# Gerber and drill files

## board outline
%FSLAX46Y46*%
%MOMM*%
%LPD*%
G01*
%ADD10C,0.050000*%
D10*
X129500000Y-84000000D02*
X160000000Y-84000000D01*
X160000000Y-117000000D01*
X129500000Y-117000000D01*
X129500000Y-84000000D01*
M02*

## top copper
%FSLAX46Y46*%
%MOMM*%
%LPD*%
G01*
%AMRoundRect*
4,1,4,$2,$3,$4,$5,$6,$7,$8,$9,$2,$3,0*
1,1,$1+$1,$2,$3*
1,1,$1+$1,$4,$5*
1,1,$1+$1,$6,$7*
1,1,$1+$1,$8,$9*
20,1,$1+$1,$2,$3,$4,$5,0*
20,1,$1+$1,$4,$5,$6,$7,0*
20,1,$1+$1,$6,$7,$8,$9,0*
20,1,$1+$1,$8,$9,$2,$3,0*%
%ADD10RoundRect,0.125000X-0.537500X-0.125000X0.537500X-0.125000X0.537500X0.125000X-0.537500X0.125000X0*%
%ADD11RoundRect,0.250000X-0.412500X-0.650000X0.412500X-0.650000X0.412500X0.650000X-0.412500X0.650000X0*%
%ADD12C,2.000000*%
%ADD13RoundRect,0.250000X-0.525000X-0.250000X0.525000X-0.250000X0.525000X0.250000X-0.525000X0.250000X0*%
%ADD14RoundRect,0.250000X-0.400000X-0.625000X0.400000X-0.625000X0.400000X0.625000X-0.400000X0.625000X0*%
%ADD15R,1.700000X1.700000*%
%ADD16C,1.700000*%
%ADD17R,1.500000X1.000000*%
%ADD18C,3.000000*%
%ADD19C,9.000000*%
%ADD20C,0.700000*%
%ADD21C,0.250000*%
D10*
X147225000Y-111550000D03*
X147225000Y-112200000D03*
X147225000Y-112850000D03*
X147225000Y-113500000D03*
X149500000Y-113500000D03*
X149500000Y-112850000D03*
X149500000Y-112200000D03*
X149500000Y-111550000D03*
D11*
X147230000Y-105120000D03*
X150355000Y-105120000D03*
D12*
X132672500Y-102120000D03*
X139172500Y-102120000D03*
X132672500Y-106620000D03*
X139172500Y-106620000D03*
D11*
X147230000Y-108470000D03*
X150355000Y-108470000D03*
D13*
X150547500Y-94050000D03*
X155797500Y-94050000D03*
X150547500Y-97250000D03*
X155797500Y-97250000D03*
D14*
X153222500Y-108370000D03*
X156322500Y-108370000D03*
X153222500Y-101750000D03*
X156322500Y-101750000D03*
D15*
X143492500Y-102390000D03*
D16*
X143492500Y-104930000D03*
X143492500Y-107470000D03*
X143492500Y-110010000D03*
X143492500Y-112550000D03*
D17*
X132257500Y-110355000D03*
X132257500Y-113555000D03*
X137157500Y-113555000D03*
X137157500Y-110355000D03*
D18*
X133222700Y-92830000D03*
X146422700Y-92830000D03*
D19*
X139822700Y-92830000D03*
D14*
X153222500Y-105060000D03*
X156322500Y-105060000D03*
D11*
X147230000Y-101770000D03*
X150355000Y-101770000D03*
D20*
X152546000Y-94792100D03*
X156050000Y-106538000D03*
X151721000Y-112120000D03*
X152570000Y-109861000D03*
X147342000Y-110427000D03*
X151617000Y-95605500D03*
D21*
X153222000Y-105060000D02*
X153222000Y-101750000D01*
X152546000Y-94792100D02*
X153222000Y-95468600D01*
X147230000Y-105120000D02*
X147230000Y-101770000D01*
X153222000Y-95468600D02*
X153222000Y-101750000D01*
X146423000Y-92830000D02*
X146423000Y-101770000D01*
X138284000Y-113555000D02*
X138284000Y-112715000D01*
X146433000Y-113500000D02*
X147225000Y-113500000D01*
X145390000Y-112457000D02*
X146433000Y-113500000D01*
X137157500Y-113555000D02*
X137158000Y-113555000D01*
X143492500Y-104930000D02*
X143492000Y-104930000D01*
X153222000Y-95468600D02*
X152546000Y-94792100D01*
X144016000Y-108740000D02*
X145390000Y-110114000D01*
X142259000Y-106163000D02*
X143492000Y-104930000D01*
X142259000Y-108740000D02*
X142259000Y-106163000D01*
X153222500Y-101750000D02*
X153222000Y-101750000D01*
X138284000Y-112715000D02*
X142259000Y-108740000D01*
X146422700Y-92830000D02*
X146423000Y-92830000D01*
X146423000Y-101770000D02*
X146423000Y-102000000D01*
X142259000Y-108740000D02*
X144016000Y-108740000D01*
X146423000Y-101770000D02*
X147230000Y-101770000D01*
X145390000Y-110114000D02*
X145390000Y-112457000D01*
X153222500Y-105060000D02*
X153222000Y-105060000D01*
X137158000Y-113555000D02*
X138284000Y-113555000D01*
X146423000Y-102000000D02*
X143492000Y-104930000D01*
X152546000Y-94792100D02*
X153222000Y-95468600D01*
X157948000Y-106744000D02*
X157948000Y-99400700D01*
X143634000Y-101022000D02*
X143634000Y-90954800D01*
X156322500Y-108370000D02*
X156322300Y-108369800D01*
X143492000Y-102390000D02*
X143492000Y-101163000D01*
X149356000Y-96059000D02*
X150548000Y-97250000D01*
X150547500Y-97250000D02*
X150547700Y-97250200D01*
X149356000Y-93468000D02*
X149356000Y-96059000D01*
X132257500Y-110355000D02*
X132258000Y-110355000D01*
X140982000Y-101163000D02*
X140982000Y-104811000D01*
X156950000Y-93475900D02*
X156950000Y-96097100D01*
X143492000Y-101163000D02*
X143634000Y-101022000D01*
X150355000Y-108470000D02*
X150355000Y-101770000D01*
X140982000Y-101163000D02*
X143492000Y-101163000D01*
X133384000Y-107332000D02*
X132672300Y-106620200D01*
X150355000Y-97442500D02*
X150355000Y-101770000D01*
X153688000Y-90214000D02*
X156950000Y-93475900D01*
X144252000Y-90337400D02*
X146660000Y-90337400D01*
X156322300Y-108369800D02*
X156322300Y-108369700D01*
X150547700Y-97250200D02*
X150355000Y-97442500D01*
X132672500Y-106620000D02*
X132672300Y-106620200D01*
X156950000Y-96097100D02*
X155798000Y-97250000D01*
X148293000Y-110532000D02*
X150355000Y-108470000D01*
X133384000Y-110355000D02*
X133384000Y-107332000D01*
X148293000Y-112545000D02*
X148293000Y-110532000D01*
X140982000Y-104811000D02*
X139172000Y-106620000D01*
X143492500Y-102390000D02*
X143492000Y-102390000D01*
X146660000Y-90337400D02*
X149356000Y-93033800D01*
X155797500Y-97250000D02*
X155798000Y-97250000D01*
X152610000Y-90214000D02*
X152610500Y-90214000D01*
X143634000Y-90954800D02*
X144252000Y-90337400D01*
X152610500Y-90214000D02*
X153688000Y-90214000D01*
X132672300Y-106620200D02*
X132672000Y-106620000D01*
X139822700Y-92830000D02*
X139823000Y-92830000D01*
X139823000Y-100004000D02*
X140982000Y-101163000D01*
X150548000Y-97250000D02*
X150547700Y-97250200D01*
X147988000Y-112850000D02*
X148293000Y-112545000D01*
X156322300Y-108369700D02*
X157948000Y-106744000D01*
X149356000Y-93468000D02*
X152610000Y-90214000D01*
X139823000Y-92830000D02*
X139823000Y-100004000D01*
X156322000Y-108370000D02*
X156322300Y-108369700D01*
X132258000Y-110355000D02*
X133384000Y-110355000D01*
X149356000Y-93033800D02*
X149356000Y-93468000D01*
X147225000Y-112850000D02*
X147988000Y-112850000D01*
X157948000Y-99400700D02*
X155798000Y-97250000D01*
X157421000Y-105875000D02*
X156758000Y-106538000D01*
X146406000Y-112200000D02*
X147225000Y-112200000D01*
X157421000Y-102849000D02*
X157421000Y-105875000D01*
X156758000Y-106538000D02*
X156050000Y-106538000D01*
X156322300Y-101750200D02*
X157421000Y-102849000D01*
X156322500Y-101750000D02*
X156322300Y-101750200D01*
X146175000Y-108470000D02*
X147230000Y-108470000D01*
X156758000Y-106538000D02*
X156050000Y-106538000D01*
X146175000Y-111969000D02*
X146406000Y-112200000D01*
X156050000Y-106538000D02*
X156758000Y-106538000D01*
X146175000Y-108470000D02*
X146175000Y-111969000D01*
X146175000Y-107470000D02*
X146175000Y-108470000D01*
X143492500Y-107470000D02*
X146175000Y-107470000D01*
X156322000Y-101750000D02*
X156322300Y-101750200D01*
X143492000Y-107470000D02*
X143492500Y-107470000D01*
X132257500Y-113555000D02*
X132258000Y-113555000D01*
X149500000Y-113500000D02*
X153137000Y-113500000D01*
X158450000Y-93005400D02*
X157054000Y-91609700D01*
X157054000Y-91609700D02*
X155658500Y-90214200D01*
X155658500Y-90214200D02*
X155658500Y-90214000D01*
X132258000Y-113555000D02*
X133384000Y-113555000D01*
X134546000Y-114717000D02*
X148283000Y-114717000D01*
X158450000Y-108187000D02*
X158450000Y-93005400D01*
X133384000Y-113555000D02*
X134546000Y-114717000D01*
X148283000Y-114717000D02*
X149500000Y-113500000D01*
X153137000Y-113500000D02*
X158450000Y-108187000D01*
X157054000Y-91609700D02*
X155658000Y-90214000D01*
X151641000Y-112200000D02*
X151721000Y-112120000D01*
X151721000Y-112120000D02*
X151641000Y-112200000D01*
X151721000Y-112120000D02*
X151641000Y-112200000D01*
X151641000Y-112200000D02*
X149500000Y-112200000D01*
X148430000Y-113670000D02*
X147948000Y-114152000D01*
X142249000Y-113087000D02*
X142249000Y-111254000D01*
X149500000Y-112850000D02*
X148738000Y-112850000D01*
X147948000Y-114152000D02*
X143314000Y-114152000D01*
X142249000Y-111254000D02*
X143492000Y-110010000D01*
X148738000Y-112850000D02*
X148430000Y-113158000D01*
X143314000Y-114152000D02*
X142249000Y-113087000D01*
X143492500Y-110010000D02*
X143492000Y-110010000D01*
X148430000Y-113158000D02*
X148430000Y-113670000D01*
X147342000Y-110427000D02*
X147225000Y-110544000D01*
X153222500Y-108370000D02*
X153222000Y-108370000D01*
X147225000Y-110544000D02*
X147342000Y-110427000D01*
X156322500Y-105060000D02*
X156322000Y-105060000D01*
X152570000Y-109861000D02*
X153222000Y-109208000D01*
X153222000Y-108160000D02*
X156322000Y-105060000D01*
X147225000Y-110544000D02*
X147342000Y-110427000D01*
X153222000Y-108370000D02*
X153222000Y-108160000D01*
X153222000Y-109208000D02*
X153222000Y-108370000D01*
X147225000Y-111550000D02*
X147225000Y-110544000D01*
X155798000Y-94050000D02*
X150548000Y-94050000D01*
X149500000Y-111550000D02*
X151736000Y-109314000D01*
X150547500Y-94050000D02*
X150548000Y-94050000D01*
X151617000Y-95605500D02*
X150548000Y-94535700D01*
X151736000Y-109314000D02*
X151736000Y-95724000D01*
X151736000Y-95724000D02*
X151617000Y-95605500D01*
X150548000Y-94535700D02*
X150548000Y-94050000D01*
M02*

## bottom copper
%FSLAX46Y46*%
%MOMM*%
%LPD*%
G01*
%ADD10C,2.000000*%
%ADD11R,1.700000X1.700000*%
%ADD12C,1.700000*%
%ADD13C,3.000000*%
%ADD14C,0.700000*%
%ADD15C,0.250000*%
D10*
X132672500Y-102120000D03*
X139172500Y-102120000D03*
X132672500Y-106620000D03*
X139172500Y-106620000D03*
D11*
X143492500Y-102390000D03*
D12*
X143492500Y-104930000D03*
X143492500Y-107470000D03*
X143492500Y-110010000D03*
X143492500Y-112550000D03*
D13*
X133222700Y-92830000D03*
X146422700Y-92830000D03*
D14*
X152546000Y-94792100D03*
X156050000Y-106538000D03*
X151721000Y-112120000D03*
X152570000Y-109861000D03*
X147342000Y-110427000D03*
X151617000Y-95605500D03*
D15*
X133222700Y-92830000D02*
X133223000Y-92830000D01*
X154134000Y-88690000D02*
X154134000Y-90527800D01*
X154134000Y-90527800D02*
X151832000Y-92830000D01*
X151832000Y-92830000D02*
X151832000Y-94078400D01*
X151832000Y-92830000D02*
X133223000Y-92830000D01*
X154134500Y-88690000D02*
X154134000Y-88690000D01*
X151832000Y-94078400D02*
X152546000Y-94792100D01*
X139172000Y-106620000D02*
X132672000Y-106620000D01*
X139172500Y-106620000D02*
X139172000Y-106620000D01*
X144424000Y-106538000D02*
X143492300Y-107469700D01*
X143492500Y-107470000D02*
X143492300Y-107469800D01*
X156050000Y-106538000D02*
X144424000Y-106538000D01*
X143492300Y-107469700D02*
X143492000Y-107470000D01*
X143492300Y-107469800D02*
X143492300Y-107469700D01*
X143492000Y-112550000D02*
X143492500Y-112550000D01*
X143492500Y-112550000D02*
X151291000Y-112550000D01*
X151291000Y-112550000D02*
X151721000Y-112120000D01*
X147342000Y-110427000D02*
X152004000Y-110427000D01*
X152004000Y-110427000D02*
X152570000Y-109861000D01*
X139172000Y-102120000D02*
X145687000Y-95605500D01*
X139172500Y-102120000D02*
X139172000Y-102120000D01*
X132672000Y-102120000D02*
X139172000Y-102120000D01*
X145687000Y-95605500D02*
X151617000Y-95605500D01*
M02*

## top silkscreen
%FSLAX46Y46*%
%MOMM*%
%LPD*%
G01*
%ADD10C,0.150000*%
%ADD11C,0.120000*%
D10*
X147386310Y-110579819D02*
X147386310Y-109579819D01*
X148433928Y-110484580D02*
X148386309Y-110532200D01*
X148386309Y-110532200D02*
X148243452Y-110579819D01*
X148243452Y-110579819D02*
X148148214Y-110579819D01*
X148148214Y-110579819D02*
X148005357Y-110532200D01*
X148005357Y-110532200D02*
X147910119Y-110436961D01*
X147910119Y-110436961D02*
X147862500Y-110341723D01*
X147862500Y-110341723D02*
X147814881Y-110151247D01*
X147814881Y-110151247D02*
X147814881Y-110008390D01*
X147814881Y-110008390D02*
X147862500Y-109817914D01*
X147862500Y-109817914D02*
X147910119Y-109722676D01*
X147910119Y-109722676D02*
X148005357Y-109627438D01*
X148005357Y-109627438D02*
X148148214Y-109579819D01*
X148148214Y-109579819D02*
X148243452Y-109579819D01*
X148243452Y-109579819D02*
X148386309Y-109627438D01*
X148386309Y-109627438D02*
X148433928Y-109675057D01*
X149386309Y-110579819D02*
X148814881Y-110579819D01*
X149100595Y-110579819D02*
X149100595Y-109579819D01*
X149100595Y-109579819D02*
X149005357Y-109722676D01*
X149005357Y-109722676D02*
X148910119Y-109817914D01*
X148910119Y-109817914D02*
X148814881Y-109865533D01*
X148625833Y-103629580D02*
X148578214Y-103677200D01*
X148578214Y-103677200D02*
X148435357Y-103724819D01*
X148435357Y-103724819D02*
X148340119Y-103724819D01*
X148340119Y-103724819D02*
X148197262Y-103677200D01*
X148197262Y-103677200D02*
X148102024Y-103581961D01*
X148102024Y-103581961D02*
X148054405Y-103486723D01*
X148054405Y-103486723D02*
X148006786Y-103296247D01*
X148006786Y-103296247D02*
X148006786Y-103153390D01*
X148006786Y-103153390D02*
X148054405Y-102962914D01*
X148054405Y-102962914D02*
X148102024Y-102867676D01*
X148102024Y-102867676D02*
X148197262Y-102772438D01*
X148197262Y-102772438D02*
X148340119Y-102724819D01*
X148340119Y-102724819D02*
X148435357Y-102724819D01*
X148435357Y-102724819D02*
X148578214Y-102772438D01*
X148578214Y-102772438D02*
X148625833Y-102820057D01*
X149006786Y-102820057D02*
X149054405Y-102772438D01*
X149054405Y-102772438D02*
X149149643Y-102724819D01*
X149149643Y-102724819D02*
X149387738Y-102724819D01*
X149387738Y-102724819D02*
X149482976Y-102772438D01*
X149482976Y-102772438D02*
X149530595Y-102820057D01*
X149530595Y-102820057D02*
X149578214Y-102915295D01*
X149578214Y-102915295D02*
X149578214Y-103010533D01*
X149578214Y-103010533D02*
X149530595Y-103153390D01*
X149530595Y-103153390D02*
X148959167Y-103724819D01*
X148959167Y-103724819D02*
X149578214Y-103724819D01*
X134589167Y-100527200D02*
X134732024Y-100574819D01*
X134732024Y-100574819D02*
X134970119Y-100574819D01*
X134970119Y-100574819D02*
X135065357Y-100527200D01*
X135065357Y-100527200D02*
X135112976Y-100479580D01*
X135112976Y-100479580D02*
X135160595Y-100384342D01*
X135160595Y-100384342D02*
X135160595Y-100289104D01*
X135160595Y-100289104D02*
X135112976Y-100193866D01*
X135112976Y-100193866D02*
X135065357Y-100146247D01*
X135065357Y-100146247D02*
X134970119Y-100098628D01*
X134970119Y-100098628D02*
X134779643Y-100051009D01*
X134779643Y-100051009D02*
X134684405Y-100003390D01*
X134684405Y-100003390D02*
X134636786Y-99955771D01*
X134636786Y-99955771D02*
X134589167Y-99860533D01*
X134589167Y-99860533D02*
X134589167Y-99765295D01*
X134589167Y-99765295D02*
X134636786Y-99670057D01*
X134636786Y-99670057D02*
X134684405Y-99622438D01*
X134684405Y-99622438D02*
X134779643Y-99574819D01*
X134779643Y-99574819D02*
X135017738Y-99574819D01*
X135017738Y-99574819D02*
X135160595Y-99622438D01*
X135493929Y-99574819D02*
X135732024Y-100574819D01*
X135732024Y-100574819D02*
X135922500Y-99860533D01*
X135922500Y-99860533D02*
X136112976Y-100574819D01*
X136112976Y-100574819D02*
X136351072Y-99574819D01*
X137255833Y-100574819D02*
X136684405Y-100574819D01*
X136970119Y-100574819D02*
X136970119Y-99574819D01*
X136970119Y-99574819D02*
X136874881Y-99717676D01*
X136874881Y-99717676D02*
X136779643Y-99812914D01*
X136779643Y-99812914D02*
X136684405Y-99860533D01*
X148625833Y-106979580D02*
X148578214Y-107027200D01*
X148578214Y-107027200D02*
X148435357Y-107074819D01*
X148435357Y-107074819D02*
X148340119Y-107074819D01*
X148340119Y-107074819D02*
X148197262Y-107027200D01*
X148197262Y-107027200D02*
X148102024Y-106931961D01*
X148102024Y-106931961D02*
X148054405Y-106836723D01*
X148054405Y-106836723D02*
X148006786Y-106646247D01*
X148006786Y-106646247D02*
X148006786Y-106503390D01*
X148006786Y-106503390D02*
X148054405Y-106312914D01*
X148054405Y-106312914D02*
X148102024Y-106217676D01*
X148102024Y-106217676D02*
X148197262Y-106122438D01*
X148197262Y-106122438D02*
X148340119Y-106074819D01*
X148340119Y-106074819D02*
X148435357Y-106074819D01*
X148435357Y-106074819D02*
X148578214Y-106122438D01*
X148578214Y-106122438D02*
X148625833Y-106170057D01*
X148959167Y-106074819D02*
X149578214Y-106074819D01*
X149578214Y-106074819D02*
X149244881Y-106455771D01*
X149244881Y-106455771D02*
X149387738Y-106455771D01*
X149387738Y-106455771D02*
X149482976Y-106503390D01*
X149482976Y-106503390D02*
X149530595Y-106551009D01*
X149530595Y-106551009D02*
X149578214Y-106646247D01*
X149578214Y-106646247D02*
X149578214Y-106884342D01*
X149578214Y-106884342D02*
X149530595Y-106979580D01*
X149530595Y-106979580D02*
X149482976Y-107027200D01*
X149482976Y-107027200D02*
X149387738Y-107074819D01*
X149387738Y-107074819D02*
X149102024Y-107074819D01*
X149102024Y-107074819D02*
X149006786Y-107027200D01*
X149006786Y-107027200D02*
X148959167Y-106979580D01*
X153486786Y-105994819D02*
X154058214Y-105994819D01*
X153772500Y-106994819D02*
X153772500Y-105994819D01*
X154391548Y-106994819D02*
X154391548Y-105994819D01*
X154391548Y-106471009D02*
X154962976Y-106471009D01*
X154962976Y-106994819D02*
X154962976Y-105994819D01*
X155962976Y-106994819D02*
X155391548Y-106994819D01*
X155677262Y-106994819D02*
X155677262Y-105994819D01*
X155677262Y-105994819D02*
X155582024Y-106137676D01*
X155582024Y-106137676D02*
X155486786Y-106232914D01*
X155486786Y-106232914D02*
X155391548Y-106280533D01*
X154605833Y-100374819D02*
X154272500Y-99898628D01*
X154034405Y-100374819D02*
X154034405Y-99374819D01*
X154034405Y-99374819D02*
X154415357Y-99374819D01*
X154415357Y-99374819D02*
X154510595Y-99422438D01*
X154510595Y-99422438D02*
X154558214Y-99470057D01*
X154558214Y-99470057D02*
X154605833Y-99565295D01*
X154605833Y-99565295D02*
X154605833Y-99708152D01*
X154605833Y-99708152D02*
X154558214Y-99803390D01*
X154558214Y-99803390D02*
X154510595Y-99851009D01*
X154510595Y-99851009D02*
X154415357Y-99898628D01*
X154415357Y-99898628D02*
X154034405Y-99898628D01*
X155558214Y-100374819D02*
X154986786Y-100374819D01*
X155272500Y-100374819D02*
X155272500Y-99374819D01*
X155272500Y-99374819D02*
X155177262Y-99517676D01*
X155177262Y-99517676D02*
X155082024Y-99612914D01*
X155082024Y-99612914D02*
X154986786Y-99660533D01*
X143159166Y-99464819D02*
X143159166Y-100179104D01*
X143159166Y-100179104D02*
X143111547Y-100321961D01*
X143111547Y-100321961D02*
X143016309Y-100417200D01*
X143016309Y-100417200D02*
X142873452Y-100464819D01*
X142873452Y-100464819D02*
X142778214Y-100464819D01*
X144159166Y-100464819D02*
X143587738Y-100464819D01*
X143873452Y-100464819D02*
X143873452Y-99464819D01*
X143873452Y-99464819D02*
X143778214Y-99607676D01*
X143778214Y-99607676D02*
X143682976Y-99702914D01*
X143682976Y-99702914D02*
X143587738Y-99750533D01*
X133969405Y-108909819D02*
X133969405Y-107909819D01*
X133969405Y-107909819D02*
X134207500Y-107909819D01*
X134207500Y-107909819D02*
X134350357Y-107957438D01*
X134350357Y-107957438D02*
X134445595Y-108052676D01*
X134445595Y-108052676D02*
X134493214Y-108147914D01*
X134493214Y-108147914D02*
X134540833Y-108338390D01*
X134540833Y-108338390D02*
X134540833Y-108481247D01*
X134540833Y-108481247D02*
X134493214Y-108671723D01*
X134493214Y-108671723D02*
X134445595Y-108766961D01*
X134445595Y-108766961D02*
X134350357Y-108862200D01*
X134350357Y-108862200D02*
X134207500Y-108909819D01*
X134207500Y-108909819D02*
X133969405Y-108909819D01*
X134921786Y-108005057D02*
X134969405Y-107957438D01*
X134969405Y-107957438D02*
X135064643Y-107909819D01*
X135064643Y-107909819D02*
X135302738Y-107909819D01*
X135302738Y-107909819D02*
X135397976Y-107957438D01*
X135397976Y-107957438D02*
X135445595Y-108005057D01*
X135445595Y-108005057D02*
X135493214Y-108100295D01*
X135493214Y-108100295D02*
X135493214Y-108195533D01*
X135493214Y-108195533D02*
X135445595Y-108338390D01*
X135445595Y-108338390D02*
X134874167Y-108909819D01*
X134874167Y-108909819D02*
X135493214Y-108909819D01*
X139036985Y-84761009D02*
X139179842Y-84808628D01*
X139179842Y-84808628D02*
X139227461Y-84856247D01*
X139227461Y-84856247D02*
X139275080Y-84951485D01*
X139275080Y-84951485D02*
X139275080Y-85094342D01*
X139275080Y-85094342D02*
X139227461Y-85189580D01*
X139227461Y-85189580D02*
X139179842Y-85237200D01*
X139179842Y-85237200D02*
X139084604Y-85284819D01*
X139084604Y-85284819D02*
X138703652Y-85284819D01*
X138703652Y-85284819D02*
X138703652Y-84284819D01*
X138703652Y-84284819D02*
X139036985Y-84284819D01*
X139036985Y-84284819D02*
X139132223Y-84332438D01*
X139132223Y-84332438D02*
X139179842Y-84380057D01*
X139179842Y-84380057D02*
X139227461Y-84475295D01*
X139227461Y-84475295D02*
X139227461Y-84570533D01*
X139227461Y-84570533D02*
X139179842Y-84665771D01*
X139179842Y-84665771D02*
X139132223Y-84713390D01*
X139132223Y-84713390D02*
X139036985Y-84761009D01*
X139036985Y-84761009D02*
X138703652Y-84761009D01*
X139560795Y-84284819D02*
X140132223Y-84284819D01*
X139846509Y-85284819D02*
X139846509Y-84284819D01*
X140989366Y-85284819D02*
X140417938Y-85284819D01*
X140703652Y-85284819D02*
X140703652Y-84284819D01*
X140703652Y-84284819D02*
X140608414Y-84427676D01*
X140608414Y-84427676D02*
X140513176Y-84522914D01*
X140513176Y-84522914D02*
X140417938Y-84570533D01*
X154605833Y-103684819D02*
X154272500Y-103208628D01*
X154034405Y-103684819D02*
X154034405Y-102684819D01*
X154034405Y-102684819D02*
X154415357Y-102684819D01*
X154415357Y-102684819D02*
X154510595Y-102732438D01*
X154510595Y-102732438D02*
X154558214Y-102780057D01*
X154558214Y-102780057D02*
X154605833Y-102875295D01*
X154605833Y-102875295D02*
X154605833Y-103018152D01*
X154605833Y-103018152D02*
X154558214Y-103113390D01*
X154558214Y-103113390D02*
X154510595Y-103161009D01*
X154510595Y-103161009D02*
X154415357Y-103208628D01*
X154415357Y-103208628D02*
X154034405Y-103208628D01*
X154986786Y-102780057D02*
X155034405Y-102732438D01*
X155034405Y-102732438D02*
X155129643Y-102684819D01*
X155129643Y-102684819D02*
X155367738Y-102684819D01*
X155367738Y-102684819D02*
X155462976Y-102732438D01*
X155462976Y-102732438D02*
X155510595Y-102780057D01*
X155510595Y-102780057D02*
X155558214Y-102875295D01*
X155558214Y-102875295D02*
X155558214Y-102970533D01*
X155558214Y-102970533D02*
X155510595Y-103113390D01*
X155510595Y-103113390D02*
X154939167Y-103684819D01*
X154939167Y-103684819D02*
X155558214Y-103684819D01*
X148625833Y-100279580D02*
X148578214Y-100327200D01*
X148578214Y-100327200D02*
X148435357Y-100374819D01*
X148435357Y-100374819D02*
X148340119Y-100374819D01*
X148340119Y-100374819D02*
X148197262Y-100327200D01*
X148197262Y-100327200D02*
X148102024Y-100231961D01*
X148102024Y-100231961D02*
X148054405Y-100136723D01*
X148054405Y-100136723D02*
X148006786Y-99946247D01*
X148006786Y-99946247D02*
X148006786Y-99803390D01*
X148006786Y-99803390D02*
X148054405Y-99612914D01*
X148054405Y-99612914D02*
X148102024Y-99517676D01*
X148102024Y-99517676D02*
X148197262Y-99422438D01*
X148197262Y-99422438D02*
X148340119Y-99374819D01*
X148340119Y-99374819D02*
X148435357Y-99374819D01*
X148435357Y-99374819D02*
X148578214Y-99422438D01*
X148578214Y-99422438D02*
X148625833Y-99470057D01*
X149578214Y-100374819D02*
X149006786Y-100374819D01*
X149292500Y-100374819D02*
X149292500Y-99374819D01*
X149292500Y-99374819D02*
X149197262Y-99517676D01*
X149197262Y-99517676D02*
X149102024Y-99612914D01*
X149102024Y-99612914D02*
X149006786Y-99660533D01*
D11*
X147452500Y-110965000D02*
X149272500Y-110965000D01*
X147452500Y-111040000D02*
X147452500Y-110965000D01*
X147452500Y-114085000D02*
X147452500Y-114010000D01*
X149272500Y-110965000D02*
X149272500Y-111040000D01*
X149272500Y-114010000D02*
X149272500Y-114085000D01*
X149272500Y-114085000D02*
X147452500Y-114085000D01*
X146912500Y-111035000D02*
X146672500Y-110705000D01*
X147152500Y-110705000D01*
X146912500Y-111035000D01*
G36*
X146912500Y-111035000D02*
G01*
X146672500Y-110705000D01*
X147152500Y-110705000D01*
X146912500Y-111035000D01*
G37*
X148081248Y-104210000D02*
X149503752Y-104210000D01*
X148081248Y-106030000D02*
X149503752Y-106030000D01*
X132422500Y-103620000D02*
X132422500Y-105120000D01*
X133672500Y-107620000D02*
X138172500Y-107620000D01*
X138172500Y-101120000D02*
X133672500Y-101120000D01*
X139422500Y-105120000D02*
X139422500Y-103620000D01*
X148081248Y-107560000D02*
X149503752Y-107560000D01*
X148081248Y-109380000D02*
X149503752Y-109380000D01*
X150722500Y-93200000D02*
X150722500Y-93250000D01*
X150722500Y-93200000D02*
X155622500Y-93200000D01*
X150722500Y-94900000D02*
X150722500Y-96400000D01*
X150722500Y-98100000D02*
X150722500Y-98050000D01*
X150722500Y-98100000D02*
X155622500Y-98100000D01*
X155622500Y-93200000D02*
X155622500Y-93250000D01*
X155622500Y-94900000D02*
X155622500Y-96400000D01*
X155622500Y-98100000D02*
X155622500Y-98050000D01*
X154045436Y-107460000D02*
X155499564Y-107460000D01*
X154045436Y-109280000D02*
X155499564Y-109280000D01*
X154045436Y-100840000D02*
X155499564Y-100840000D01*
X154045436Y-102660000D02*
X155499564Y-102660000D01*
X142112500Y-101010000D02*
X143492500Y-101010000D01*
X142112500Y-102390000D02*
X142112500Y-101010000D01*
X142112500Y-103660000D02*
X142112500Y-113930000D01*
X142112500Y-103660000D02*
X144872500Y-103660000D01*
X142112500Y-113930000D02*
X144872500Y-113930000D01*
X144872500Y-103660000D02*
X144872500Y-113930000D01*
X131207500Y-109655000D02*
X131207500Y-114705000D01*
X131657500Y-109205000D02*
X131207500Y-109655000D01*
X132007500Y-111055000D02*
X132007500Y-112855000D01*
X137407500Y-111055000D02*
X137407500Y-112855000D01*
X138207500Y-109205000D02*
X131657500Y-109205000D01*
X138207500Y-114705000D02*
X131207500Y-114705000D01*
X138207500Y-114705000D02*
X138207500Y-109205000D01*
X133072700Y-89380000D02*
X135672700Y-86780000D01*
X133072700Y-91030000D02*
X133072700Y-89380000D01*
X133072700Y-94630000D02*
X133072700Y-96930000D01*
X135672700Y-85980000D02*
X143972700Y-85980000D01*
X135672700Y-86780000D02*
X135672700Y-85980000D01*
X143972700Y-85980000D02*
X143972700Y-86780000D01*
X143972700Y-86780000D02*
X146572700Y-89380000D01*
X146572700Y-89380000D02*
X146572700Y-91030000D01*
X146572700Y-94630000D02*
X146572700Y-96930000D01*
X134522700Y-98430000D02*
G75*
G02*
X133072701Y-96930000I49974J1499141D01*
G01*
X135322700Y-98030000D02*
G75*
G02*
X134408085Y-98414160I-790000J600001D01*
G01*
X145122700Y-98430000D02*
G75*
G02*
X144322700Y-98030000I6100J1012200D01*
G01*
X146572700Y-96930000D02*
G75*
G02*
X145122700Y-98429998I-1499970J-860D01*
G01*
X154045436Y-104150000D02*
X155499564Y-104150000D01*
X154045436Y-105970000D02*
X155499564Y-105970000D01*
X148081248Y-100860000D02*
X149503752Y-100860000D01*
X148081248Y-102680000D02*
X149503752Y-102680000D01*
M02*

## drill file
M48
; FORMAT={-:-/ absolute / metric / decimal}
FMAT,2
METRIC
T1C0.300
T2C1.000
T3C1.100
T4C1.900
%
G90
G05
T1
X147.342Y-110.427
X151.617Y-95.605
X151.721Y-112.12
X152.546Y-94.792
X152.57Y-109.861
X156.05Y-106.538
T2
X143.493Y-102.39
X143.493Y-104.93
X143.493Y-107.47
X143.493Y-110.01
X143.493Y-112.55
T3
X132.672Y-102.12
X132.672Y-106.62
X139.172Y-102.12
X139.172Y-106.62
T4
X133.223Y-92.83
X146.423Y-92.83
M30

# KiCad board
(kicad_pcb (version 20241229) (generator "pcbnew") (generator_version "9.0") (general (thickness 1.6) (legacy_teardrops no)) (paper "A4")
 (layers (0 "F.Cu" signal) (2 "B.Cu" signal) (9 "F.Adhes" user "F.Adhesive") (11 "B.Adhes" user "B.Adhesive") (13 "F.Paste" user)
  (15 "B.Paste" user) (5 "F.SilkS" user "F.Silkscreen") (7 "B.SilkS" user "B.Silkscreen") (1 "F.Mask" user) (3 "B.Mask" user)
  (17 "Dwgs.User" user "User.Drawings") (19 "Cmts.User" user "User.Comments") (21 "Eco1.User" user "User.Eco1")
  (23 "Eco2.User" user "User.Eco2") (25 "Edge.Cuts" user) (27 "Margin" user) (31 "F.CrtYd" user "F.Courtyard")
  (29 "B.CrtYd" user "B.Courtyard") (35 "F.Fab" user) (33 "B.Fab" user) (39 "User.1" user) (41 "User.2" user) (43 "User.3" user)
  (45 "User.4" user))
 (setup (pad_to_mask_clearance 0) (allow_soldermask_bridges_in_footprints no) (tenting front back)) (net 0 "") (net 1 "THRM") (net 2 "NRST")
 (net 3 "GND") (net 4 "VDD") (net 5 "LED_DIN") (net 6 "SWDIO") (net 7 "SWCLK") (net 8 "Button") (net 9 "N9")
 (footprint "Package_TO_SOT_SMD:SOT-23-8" (layer "F.Cu") (at 148.3625 112.525)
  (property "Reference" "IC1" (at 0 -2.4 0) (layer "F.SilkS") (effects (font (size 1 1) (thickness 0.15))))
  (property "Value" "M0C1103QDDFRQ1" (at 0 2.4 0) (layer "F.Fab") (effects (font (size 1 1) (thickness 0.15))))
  (fp_line (start -0.91 -1.56) (end 0.91 -1.56) (stroke (width 0.12) (type solid)) (layer "F.SilkS"))
  (fp_line (start -0.91 -1.485) (end -0.91 -1.56) (stroke (width 0.12) (type solid)) (layer "F.SilkS"))
  (fp_line (start -0.91 1.56) (end -0.91 1.485) (stroke (width 0.12) (type solid)) (layer "F.SilkS"))
  (fp_line (start 0.91 -1.56) (end 0.91 -1.485) (stroke (width 0.12) (type solid)) (layer "F.SilkS"))
  (fp_line (start 0.91 1.485) (end 0.91 1.56) (stroke (width 0.12) (type solid)) (layer "F.SilkS"))
  (fp_line (start 0.91 1.56) (end -0.91 1.56) (stroke (width 0.12) (type solid)) (layer "F.SilkS"))
  (fp_poly (pts (xy -1.45 -1.49) (xy -1.69 -1.82) (xy -1.21 -1.82)) (stroke (width 0.12) (type solid)) (fill yes) (layer "F.SilkS"))
  (pad "1" smd roundrect (at -1.1375 -0.975) (size 1.325 0.5) (layers "F.Cu" "F.Mask" "F.Paste") (roundrect_rratio 0.25) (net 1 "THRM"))
  (pad "2" smd roundrect (at -1.1375 -0.325) (size 1.325 0.5) (layers "F.Cu" "F.Mask" "F.Paste") (roundrect_rratio 0.25) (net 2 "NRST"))
  (pad "3" smd roundrect (at -1.1375 0.325) (size 1.325 0.5) (layers "F.Cu" "F.Mask" "F.Paste") (roundrect_rratio 0.25) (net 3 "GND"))
  (pad "4" smd roundrect (at -1.1375 0.975) (size 1.325 0.5) (layers "F.Cu" "F.Mask" "F.Paste") (roundrect_rratio 0.25) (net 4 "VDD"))
  (pad "5" smd roundrect (at 1.1375 0.975) (size 1.325 0.5) (layers "F.Cu" "F.Mask" "F.Paste") (roundrect_rratio 0.25) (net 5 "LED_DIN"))
  (pad "6" smd roundrect (at 1.1375 0.325) (size 1.325 0.5) (layers "F.Cu" "F.Mask" "F.Paste") (roundrect_rratio 0.25) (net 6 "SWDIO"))
  (pad "7" smd roundrect (at 1.1375 -0.325) (size 1.325 0.5) (layers "F.Cu" "F.Mask" "F.Paste") (roundrect_rratio 0.25) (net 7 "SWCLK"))
  (pad "8" smd roundrect (at 1.1375 -0.975) (size 1.325 0.5) (layers "F.Cu" "F.Mask" "F.Paste") (roundrect_rratio 0.25) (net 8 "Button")))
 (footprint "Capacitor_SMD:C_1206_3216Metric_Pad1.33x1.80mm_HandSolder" (layer "F.Cu") (at 148.7925 105.12)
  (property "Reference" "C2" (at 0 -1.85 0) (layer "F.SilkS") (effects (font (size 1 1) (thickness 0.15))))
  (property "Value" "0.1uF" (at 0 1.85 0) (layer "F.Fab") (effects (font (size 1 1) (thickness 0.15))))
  (fp_line (start -0.711252 -0.91) (end 0.711252 -0.91) (stroke (width 0.12) (type solid)) (layer "F.SilkS"))
  (fp_line (start -0.711252 0.91) (end 0.711252 0.91) (stroke (width 0.12) (type solid)) (layer "F.SilkS"))
  (pad "1" smd roundrect (at -1.5625 0) (size 1.325 1.8) (layers "F.Cu" "F.Mask" "F.Paste") (roundrect_rratio 0.188679) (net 4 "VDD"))
  (pad "2" smd roundrect (at 1.5625 0) (size 1.325 1.8) (layers "F.Cu" "F.Mask" "F.Paste") (roundrect_rratio 0.188679) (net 3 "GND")))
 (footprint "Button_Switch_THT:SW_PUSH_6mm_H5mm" (layer "F.Cu") (at 132.6725 102.12)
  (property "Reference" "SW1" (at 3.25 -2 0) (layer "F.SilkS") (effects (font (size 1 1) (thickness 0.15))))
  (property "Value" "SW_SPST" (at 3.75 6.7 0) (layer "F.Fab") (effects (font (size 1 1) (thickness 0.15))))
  (fp_line (start -0.25 1.5) (end -0.25 3) (stroke (width 0.12) (type solid)) (layer "F.SilkS"))
  (fp_line (start 1 5.5) (end 5.5 5.5) (stroke (width 0.12) (type solid)) (layer "F.SilkS"))
  (fp_line (start 5.5 -1) (end 1 -1) (stroke (width 0.12) (type solid)) (layer "F.SilkS"))
  (fp_line (start 6.75 3) (end 6.75 1.5) (stroke (width 0.12) (type solid)) (layer "F.SilkS"))
  (pad "1" thru_hole circle (at 0 0 90) (size 2 2) (drill 1.1) (layers "*.Cu" "*.Mask") (remove_unused_layers no) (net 8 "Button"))
  (pad "1" thru_hole circle (at 6.5 0 90) (size 2 2) (drill 1.1) (layers "*.Cu" "*.Mask") (remove_unused_layers no) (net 8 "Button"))
  (pad "2" thru_hole circle (at 0 4.5 90) (size 2 2) (drill 1.1) (layers "*.Cu" "*.Mask") (remove_unused_layers no) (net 3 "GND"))
  (pad "2" thru_hole circle (at 6.5 4.5 90) (size 2 2) (drill 1.1) (layers "*.Cu" "*.Mask") (remove_unused_layers no) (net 3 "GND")))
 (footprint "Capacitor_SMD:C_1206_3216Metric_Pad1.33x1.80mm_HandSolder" (layer "F.Cu") (at 148.7925 108.47)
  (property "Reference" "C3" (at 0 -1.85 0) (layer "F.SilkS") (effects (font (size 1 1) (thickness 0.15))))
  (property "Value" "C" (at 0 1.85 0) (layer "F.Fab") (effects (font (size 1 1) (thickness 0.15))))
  (fp_line (start -0.711252 -0.91) (end 0.711252 -0.91) (stroke (width 0.12) (type solid)) (layer "F.SilkS"))
  (fp_line (start -0.711252 0.91) (end 0.711252 0.91) (stroke (width 0.12) (type solid)) (layer "F.SilkS"))
  (pad "1" smd roundrect (at -1.5625 0) (size 1.325 1.8) (layers "F.Cu" "F.Mask" "F.Paste") (roundrect_rratio 0.188679) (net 2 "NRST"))
  (pad "2" smd roundrect (at 1.5625 0) (size 1.325 1.8) (layers "F.Cu" "F.Mask" "F.Paste") (roundrect_rratio 0.188679) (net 3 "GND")))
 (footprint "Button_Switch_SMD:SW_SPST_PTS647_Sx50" (layer "F.Cu") (at 153.1725 95.65)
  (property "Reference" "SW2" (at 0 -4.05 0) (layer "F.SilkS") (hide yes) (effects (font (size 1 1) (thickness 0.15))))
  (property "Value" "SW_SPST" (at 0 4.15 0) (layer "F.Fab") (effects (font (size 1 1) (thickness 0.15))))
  (fp_line (start -2.45 -2.45) (end -2.45 -2.4) (stroke (width 0.12) (type solid)) (layer "F.SilkS"))
  (fp_line (start -2.45 -2.45) (end 2.45 -2.45) (stroke (width 0.12) (type solid)) (layer "F.SilkS"))
  (fp_line (start -2.45 -0.75) (end -2.45 0.75) (stroke (width 0.12) (type solid)) (layer "F.SilkS"))
  (fp_line (start -2.45 2.45) (end -2.45 2.4) (stroke (width 0.12) (type solid)) (layer "F.SilkS"))
  (fp_line (start -2.45 2.45) (end 2.45 2.45) (stroke (width 0.12) (type solid)) (layer "F.SilkS"))
  (fp_line (start 2.45 -2.45) (end 2.45 -2.4) (stroke (width 0.12) (type solid)) (layer "F.SilkS"))
  (fp_line (start 2.45 -0.75) (end 2.45 0.75) (stroke (width 0.12) (type solid)) (layer "F.SilkS"))
  (fp_line (start 2.45 2.45) (end 2.45 2.4) (stroke (width 0.12) (type solid)) (layer "F.SilkS"))
  (pad "1" smd roundrect (at -2.625 -1.6) (size 1.55 1) (layers "F.Cu" "F.Mask" "F.Paste") (roundrect_rratio 0.25) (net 8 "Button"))
  (pad "1" smd roundrect (at 2.625 -1.6) (size 1.55 1) (layers "F.Cu" "F.Mask" "F.Paste") (roundrect_rratio 0.25) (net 8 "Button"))
  (pad "2" smd roundrect (at -2.625 1.6) (size 1.55 1) (layers "F.Cu" "F.Mask" "F.Paste") (roundrect_rratio 0.25) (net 3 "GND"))
  (pad "2" smd roundrect (at 2.625 1.6) (size 1.55 1) (layers "F.Cu" "F.Mask" "F.Paste") (roundrect_rratio 0.25) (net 3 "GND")))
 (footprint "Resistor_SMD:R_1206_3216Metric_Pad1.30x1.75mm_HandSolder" (layer "F.Cu") (at 154.7725 108.37)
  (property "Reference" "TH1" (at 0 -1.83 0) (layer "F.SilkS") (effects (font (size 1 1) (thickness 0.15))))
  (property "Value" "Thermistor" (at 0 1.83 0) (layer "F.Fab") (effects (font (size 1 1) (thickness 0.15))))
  (fp_line (start -0.727064 -0.91) (end 0.727064 -0.91) (stroke (width 0.12) (type solid)) (layer "F.SilkS"))
  (fp_line (start -0.727064 0.91) (end 0.727064 0.91) (stroke (width 0.12) (type solid)) (layer "F.SilkS"))
  (pad "1" smd roundrect (at -1.55 0) (size 1.3 1.75) (layers "F.Cu" "F.Mask" "F.Paste") (roundrect_rratio 0.192308) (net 1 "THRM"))
  (pad "2" smd roundrect (at 1.55 0) (size 1.3 1.75) (layers "F.Cu" "F.Mask" "F.Paste") (roundrect_rratio 0.192308) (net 3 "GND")))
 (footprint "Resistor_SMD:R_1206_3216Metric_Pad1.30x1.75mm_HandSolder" (layer "F.Cu") (at 154.7725 101.75)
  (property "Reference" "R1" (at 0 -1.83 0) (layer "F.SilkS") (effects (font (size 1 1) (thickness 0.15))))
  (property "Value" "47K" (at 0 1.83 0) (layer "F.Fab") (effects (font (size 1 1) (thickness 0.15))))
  (fp_line (start -0.727064 -0.91) (end 0.727064 -0.91) (stroke (width 0.12) (type solid)) (layer "F.SilkS"))
  (fp_line (start -0.727064 0.91) (end 0.727064 0.91) (stroke (width 0.12) (type solid)) (layer "F.SilkS"))
  (pad "1" smd roundrect (at -1.55 0) (size 1.3 1.75) (layers "F.Cu" "F.Mask" "F.Paste") (roundrect_rratio 0.192308) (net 4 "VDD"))
  (pad "2" smd roundrect (at 1.55 0) (size 1.3 1.75) (layers "F.Cu" "F.Mask" "F.Paste") (roundrect_rratio 0.192308) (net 2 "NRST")))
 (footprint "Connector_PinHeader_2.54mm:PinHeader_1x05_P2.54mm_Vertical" (layer "F.Cu") (at 143.4925 102.39)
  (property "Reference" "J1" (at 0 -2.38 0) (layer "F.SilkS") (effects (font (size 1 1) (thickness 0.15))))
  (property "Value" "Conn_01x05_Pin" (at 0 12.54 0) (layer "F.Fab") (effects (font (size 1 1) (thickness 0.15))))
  (fp_line (start -1.38 -1.38) (end 0 -1.38) (stroke (width 0.12) (type solid)) (layer "F.SilkS"))
  (fp_line (start -1.38 0) (end -1.38 -1.38) (stroke (width 0.12) (type solid)) (layer "F.SilkS"))
  (fp_line (start -1.38 1.27) (end -1.38 11.54) (stroke (width 0.12) (type solid)) (layer "F.SilkS"))
  (fp_line (start -1.38 1.27) (end 1.38 1.27) (stroke (width 0.12) (type solid)) (layer "F.SilkS"))
  (fp_line (start -1.38 11.54) (end 1.38 11.54) (stroke (width 0.12) (type solid)) (layer "F.SilkS"))
  (fp_line (start 1.38 1.27) (end 1.38 11.54) (stroke (width 0.12) (type solid)) (layer "F.SilkS"))
  (pad "1" thru_hole rect (at 0 0) (size 1.7 1.7) (drill 1) (layers "*.Cu" "*.Mask") (remove_unused_layers no) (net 3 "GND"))
  (pad "2" thru_hole circle (at 0 2.54) (size 1.7 1.7) (drill 1) (layers "*.Cu" "*.Mask") (remove_unused_layers no) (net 4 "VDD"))
  (pad "3" thru_hole circle (at 0 5.08) (size 1.7 1.7) (drill 1) (layers "*.Cu" "*.Mask") (remove_unused_layers no) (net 2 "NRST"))
  (pad "4" thru_hole circle (at 0 7.62) (size 1.7 1.7) (drill 1) (layers "*.Cu" "*.Mask") (remove_unused_layers no) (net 6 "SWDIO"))
  (pad "5" thru_hole circle (at 0 10.16) (size 1.7 1.7) (drill 1) (layers "*.Cu" "*.Mask") (remove_unused_layers no) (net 7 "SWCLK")))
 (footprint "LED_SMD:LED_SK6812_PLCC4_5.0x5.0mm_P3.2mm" (layer "F.Cu") (at 134.7075 111.955)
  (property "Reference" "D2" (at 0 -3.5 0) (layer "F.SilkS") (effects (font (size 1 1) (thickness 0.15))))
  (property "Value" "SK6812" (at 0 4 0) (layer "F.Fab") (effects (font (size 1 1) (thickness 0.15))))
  (fp_line (start -3.5 -2.3) (end -3.5 2.75) (stroke (width 0.12) (type default)) (layer "F.SilkS"))
  (fp_line (start -3.05 -2.75) (end -3.5 -2.3) (stroke (width 0.12) (type default)) (layer "F.SilkS"))
  (fp_line (start -2.7 -0.9) (end -2.7 0.9) (stroke (width 0.12) (type default)) (layer "F.SilkS"))
  (fp_line (start 2.7 -0.9) (end 2.7 0.9) (stroke (width 0.12) (type default)) (layer "F.SilkS"))
  (fp_line (start 3.5 -2.75) (end -3.05 -2.75) (stroke (width 0.12) (type solid)) (layer "F.SilkS"))
  (fp_line (start 3.5 2.75) (end -3.5 2.75) (stroke (width 0.12) (type solid)) (layer "F.SilkS"))
  (fp_line (start 3.5 2.75) (end 3.5 -2.75) (stroke (width 0.12) (type default)) (layer "F.SilkS"))
  (pad "1" smd rect (at -2.45 -1.6 180) (size 1.5 1) (layers "F.Cu" "F.Mask" "F.Paste") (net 3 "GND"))
  (pad "2" smd rect (at -2.45 1.6 180) (size 1.5 1) (layers "F.Cu" "F.Mask" "F.Paste") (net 5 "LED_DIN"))
  (pad "3" smd rect (at 2.45 1.6 180) (size 1.5 1) (layers "F.Cu" "F.Mask" "F.Paste") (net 4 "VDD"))
  (pad "4" smd rect (at 2.45 -1.6 180) (size 1.5 1) (layers "F.Cu" "F.Mask" "F.Paste") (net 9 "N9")))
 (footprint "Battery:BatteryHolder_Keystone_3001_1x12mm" (layer "F.Cu") (at 139.8227 92.83)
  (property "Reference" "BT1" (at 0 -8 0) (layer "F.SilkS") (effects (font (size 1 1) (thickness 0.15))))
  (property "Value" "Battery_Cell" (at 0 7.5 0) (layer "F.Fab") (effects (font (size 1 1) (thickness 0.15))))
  (fp_line (start -6.75 -3.45) (end -4.15 -6.05) (stroke (width 0.12) (type solid)) (layer "F.SilkS"))
  (fp_line (start -6.75 -1.8) (end -6.75 -3.45) (stroke (width 0.12) (type solid)) (layer "F.SilkS"))
  (fp_line (start -6.75 1.8) (end -6.75 4.1) (stroke (width 0.12) (type solid)) (layer "F.SilkS"))
  (fp_line (start -4.15 -6.85) (end 4.15 -6.85) (stroke (width 0.12) (type solid)) (layer "F.SilkS"))
  (fp_line (start -4.15 -6.05) (end -4.15 -6.85) (stroke (width 0.12) (type solid)) (layer "F.SilkS"))
  (fp_line (start 4.15 -6.85) (end 4.15 -6.05) (stroke (width 0.12) (type solid)) (layer "F.SilkS"))
  (fp_line (start 4.15 -6.05) (end 6.75 -3.45) (stroke (width 0.12) (type solid)) (layer "F.SilkS"))
  (fp_line (start 6.75 -3.45) (end 6.75 -1.8) (stroke (width 0.12) (type solid)) (layer "F.SilkS"))
  (fp_line (start 6.75 1.8) (end 6.75 4.1) (stroke (width 0.12) (type solid)) (layer "F.SilkS"))
  (fp_arc (start -5.3 5.6) (mid -6.32849 5.143374) (end -6.75 4.1) (stroke (width 0.12) (type solid)) (layer "F.SilkS"))
  (fp_arc (start -4.5 5.2) (mid -4.90584 5.514615) (end -5.414615 5.58416) (stroke (width 0.12) (type solid)) (layer "F.SilkS"))
  (fp_arc (start 5.3 5.6) (mid 4.853425 5.493151) (end 4.5 5.2) (stroke (width 0.12) (type solid)) (layer "F.SilkS"))
  (fp_arc (start 6.75 4.1) (mid 6.328491 5.143375) (end 5.3 5.6) (stroke (width 0.12) (type solid)) (layer "F.SilkS"))
  (pad "1" thru_hole circle (at -6.6 0) (size 3 3) (drill 1.9) (layers "*.Cu" "*.Mask") (remove_unused_layers no) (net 4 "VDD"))
  (pad "1" thru_hole circle (at 6.6 0) (size 3 3) (drill 1.9) (layers "*.Cu" "*.Mask") (remove_unused_layers no) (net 4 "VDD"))
  (pad "2" smd circle (at 0 0) (size 9 9) (layers "F.Cu" "F.Mask") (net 3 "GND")))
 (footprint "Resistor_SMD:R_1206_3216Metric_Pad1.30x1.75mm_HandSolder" (layer "F.Cu") (at 154.7725 105.06)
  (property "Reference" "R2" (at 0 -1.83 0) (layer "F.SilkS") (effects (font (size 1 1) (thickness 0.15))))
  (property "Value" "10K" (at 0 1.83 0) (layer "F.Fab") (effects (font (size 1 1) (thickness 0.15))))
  (fp_line (start -0.727064 -0.91) (end 0.727064 -0.91) (stroke (width 0.12) (type solid)) (layer "F.SilkS"))
  (fp_line (start -0.727064 0.91) (end 0.727064 0.91) (stroke (width 0.12) (type solid)) (layer "F.SilkS"))
  (pad "1" smd roundrect (at -1.55 0) (size 1.3 1.75) (layers "F.Cu" "F.Mask" "F.Paste") (roundrect_rratio 0.192308) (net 4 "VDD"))
  (pad "2" smd roundrect (at 1.55 0) (size 1.3 1.75) (layers "F.Cu" "F.Mask" "F.Paste") (roundrect_rratio 0.192308) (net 1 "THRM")))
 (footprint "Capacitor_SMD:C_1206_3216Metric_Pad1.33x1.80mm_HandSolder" (layer "F.Cu") (at 148.7925 101.77)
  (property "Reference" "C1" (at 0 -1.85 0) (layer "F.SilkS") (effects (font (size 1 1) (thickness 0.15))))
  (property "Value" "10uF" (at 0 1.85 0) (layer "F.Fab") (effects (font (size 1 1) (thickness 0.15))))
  (fp_line (start -0.711252 -0.91) (end 0.711252 -0.91) (stroke (width 0.12) (type solid)) (layer "F.SilkS"))
  (fp_line (start -0.711252 0.91) (end 0.711252 0.91) (stroke (width 0.12) (type solid)) (layer "F.SilkS"))
  (pad "1" smd roundrect (at -1.5625 0) (size 1.325 1.8) (layers "F.Cu" "F.Mask" "F.Paste") (roundrect_rratio 0.188679) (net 4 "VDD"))
  (pad "2" smd roundrect (at 1.5625 0) (size 1.325 1.8) (layers "F.Cu" "F.Mask" "F.Paste") (roundrect_rratio 0.188679) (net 3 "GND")))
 (gr_rect (start 129.5 84) (end 160 117) (stroke (width 0.05) (type default)) (fill no) (layer "Edge.Cuts"))
 (segment (start 153.222 105.06) (end 153.222 101.75) (width 0.25) (layer "F.Cu") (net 4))
 (segment (start 152.546 94.7921) (end 153.222 95.4686) (width 0.25) (layer "F.Cu") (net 4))
 (segment (start 147.23 105.12) (end 147.23 101.77) (width 0.25) (layer "F.Cu") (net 4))
 (segment (start 153.222 95.4686) (end 153.222 101.75) (width 0.25) (layer "F.Cu") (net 4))
 (segment (start 146.423 92.83) (end 146.423 101.77) (width 0.25) (layer "F.Cu") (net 4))
 (segment (start 138.284 113.555) (end 138.284 112.715) (width 0.25) (layer "F.Cu") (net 4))
 (segment (start 146.433 113.5) (end 147.225 113.5) (width 0.25) (layer "F.Cu") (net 4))
 (segment (start 145.39 112.457) (end 146.433 113.5) (width 0.25) (layer "F.Cu") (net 4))
 (segment (start 137.1575 113.555) (end 137.158 113.555) (width 0.25) (layer "F.Cu") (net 4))
 (segment (start 143.4925 104.93) (end 143.492 104.93) (width 0.25) (layer "F.Cu") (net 4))
 (segment (start 153.222 95.4686) (end 152.546 94.7921) (width 0.25) (layer "F.Cu") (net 4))
 (segment (start 144.016 108.74) (end 145.39 110.114) (width 0.25) (layer "F.Cu") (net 4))
 (segment (start 142.259 106.163) (end 143.492 104.93) (width 0.25) (layer "F.Cu") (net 4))
 (segment (start 142.259 108.74) (end 142.259 106.163) (width 0.25) (layer "F.Cu") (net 4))
 (segment (start 153.2225 101.75) (end 153.222 101.75) (width 0.25) (layer "F.Cu") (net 4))
 (segment (start 138.284 112.715) (end 142.259 108.74) (width 0.25) (layer "F.Cu") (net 4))
 (segment (start 146.4227 92.83) (end 146.423 92.83) (width 0.25) (layer "F.Cu") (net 4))
 (segment (start 146.423 101.77) (end 146.423 102) (width 0.25) (layer "F.Cu") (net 4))
 (segment (start 142.259 108.74) (end 144.016 108.74) (width 0.25) (layer "F.Cu") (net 4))
 (segment (start 146.423 101.77) (end 147.23 101.77) (width 0.25) (layer "F.Cu") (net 4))
 (segment (start 145.39 110.114) (end 145.39 112.457) (width 0.25) (layer "F.Cu") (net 4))
 (segment (start 153.2225 105.06) (end 153.222 105.06) (width 0.25) (layer "F.Cu") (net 4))
 (segment (start 137.158 113.555) (end 138.284 113.555) (width 0.25) (layer "F.Cu") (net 4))
 (segment (start 146.423 102) (end 143.492 104.93) (width 0.25) (layer "F.Cu") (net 4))
 (segment (start 152.546 94.7921) (end 153.222 95.4686) (width 0.25) (layer "F.Cu") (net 4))
 (via (at 152.546 94.7921) (size 0.7) (drill 0.3) (layers "F.Cu" "B.Cu") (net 4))
 (segment (start 133.2227 92.83) (end 133.223 92.83) (width 0.25) (layer "B.Cu") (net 4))
 (segment (start 154.134 88.69) (end 154.134 90.5278) (width 0.25) (layer "B.Cu") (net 4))
 (segment (start 154.134 90.5278) (end 151.832 92.83) (width 0.25) (layer "B.Cu") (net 4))
 (segment (start 151.832 92.83) (end 151.832 94.0784) (width 0.25) (layer "B.Cu") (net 4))
 (segment (start 151.832 92.83) (end 133.223 92.83) (width 0.25) (layer "B.Cu") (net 4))
 (segment (start 154.1345 88.69) (end 154.134 88.69) (width 0.25) (layer "B.Cu") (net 4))
 (segment (start 151.832 94.0784) (end 152.546 94.7921) (width 0.25) (layer "B.Cu") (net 4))
 (segment (start 157.948 106.744) (end 157.948 99.4007) (width 0.25) (layer "F.Cu") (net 3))
 (segment (start 143.634 101.022) (end 143.634 90.9548) (width 0.25) (layer "F.Cu") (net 3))
 (segment (start 156.3225 108.37) (end 156.3223 108.3698) (width 0.25) (layer "F.Cu") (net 3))
 (segment (start 143.492 102.39) (end 143.492 101.163) (width 0.25) (layer "F.Cu") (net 3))
 (segment (start 149.356 96.059) (end 150.548 97.25) (width 0.25) (layer "F.Cu") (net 3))
 (segment (start 150.5475 97.25) (end 150.5477 97.2502) (width 0.25) (layer "F.Cu") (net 3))
 (segment (start 149.356 93.468) (end 149.356 96.059) (width 0.25) (layer "F.Cu") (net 3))
 (segment (start 132.2575 110.355) (end 132.258 110.355) (width 0.25) (layer "F.Cu") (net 3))
 (segment (start 140.982 101.163) (end 140.982 104.811) (width 0.25) (layer "F.Cu") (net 3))
 (segment (start 156.95 93.4759) (end 156.95 96.0971) (width 0.25) (layer "F.Cu") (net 3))
 (segment (start 143.492 101.163) (end 143.634 101.022) (width 0.25) (layer "F.Cu") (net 3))
 (segment (start 150.355 108.47) (end 150.355 101.77) (width 0.25) (layer "F.Cu") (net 3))
 (segment (start 140.982 101.163) (end 143.492 101.163) (width 0.25) (layer "F.Cu") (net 3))
 (segment (start 133.384 107.332) (end 132.6723 106.6202) (width 0.25) (layer "F.Cu") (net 3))
 (segment (start 150.355 97.4425) (end 150.355 101.77) (width 0.25) (layer "F.Cu") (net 3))
 (segment (start 153.688 90.214) (end 156.95 93.4759) (width 0.25) (layer "F.Cu") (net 3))
 (segment (start 144.252 90.3374) (end 146.66 90.3374) (width 0.25) (layer "F.Cu") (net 3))
 (segment (start 156.3223 108.3698) (end 156.3223 108.3697) (width 0.25) (layer "F.Cu") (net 3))
 (segment (start 150.5477 97.2502) (end 150.355 97.4425) (width 0.25) (layer "F.Cu") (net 3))
 (segment (start 132.6725 106.62) (end 132.6723 106.6202) (width 0.25) (layer "F.Cu") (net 3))
 (segment (start 156.95 96.0971) (end 155.798 97.25) (width 0.25) (layer "F.Cu") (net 3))
 (segment (start 148.293 110.532) (end 150.355 108.47) (width 0.25) (layer "F.Cu") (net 3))
 (segment (start 133.384 110.355) (end 133.384 107.332) (width 0.25) (layer "F.Cu") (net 3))
 (segment (start 148.293 112.545) (end 148.293 110.532) (width 0.25) (layer "F.Cu") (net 3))
 (segment (start 140.982 104.811) (end 139.172 106.62) (width 0.25) (layer "F.Cu") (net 3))
 (segment (start 143.4925 102.39) (end 143.492 102.39) (width 0.25) (layer "F.Cu") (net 3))
 (segment (start 146.66 90.3374) (end 149.356 93.0338) (width 0.25) (layer "F.Cu") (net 3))
 (segment (start 155.7975 97.25) (end 155.798 97.25) (width 0.25) (layer "F.Cu") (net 3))
 (segment (start 152.61 90.214) (end 152.6105 90.214) (width 0.25) (layer "F.Cu") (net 3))
 (segment (start 143.634 90.9548) (end 144.252 90.3374) (width 0.25) (layer "F.Cu") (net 3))
 (segment (start 152.6105 90.214) (end 153.688 90.214) (width 0.25) (layer "F.Cu") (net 3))
 (segment (start 132.6723 106.6202) (end 132.672 106.62) (width 0.25) (layer "F.Cu") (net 3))
 (segment (start 139.8227 92.83) (end 139.823 92.83) (width 0.25) (layer "F.Cu") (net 3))
 (segment (start 139.823 100.004) (end 140.982 101.163) (width 0.25) (layer "F.Cu") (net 3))
 (segment (start 150.548 97.25) (end 150.5477 97.2502) (width 0.25) (layer "F.Cu") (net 3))
 (segment (start 147.988 112.85) (end 148.293 112.545) (width 0.25) (layer "F.Cu") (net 3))
 (segment (start 156.3223 108.3697) (end 157.948 106.744) (width 0.25) (layer "F.Cu") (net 3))
 (segment (start 149.356 93.468) (end 152.61 90.214) (width 0.25) (layer "F.Cu") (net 3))
 (segment (start 139.823 92.83) (end 139.823 100.004) (width 0.25) (layer "F.Cu") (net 3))
 (segment (start 156.322 108.37) (end 156.3223 108.3697) (width 0.25) (layer "F.Cu") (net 3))
 (segment (start 132.258 110.355) (end 133.384 110.355) (width 0.25) (layer "F.Cu") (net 3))
 (segment (start 149.356 93.0338) (end 149.356 93.468) (width 0.25) (layer "F.Cu") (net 3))
 (segment (start 147.225 112.85) (end 147.988 112.85) (width 0.25) (layer "F.Cu") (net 3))
 (segment (start 157.948 99.4007) (end 155.798 97.25) (width 0.25) (layer "F.Cu") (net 3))
 (segment (start 139.172 106.62) (end 132.672 106.62) (width 0.25) (layer "B.Cu") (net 3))
 (segment (start 139.1725 106.62) (end 139.172 106.62) (width 0.25) (layer "B.Cu") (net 3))
 (segment (start 157.421 105.875) (end 156.758 106.538) (width 0.25) (layer "F.Cu") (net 2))
 (segment (start 146.406 112.2) (end 147.225 112.2) (width 0.25) (layer "F.Cu") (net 2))
 (segment (start 157.421 102.849) (end 157.421 105.875) (width 0.25) (layer "F.Cu") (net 2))
 (segment (start 156.758 106.538) (end 156.05 106.538) (width 0.25) (layer "F.Cu") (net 2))
 (segment (start 156.3223 101.7502) (end 157.421 102.849) (width 0.25) (layer "F.Cu") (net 2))
 (segment (start 156.3225 101.75) (end 156.3223 101.7502) (width 0.25) (layer "F.Cu") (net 2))
 (segment (start 146.175 108.47) (end 147.23 108.47) (width 0.25) (layer "F.Cu") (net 2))
 (segment (start 156.758 106.538) (end 156.05 106.538) (width 0.25) (layer "F.Cu") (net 2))
 (segment (start 146.175 111.969) (end 146.406 112.2) (width 0.25) (layer "F.Cu") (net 2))
 (segment (start 156.05 106.538) (end 156.758 106.538) (width 0.25) (layer "F.Cu") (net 2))
 (segment (start 146.175 108.47) (end 146.175 111.969) (width 0.25) (layer "F.Cu") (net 2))
 (segment (start 146.175 107.47) (end 146.175 108.47) (width 0.25) (layer "F.Cu") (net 2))
 (segment (start 143.4925 107.47) (end 146.175 107.47) (width 0.25) (layer "F.Cu") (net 2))
 (segment (start 156.322 101.75) (end 156.3223 101.7502) (width 0.25) (layer "F.Cu") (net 2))
 (segment (start 143.492 107.47) (end 143.4925 107.47) (width 0.25) (layer "F.Cu") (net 2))
 (via (at 156.05 106.538) (size 0.7) (drill 0.3) (layers "F.Cu" "B.Cu") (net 2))
 (segment (start 144.424 106.538) (end 143.4923 107.4697) (width 0.25) (layer "B.Cu") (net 2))
 (segment (start 143.4925 107.47) (end 143.4923 107.4698) (width 0.25) (layer "B.Cu") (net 2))
 (segment (start 156.05 106.538) (end 144.424 106.538) (width 0.25) (layer "B.Cu") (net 2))
 (segment (start 143.4923 107.4697) (end 143.492 107.47) (width 0.25) (layer "B.Cu") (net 2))
 (segment (start 143.4923 107.4698) (end 143.4923 107.4697) (width 0.25) (layer "B.Cu") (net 2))
 (segment (start 132.2575 113.555) (end 132.258 113.555) (width 0.25) (layer "F.Cu") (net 5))
 (segment (start 149.5 113.5) (end 153.137 113.5) (width 0.25) (layer "F.Cu") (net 5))
 (segment (start 158.45 93.0054) (end 157.054 91.6097) (width 0.25) (layer "F.Cu") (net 5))
 (segment (start 157.054 91.6097) (end 155.6585 90.2142) (width 0.25) (layer "F.Cu") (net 5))
 (segment (start 155.6585 90.2142) (end 155.6585 90.214) (width 0.25) (layer "F.Cu") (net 5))
 (segment (start 132.258 113.555) (end 133.384 113.555) (width 0.25) (layer "F.Cu") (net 5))
 (segment (start 134.546 114.717) (end 148.283 114.717) (width 0.25) (layer "F.Cu") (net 5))
 (segment (start 158.45 108.187) (end 158.45 93.0054) (width 0.25) (layer "F.Cu") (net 5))
 (segment (start 133.384 113.555) (end 134.546 114.717) (width 0.25) (layer "F.Cu") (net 5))
 (segment (start 148.283 114.717) (end 149.5 113.5) (width 0.25) (layer "F.Cu") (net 5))
 (segment (start 153.137 113.5) (end 158.45 108.187) (width 0.25) (layer "F.Cu") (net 5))
 (segment (start 157.054 91.6097) (end 155.658 90.214) (width 0.25) (layer "F.Cu") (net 5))
 (segment (start 151.641 112.2) (end 151.721 112.12) (width 0.25) (layer "F.Cu") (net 7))
 (segment (start 151.721 112.12) (end 151.641 112.2) (width 0.25) (layer "F.Cu") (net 7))
 (segment (start 151.721 112.12) (end 151.641 112.2) (width 0.25) (layer "F.Cu") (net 7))
 (segment (start 151.641 112.2) (end 149.5 112.2) (width 0.25) (layer "F.Cu") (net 7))
 (via (at 151.721 112.12) (size 0.7) (drill 0.3) (layers "F.Cu" "B.Cu") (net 7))
 (segment (start 143.492 112.55) (end 143.4925 112.55) (width 0.25) (layer "B.Cu") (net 7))
 (segment (start 143.4925 112.55) (end 151.291 112.55) (width 0.25) (layer "B.Cu") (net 7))
 (segment (start 151.291 112.55) (end 151.721 112.12) (width 0.25) (layer "B.Cu") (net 7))
 (segment (start 148.43 113.67) (end 147.948 114.152) (width 0.25) (layer "F.Cu") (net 6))
 (segment (start 142.249 113.087) (end 142.249 111.254) (width 0.25) (layer "F.Cu") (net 6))
 (segment (start 149.5 112.85) (end 148.738 112.85) (width 0.25) (layer "F.Cu") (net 6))
 (segment (start 147.948 114.152) (end 143.314 114.152) (width 0.25) (layer "F.Cu") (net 6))
 (segment (start 142.249 111.254) (end 143.492 110.01) (width 0.25) (layer "F.Cu") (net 6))
 (segment (start 148.738 112.85) (end 148.43 113.158) (width 0.25) (layer "F.Cu") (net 6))
 (segment (start 143.314 114.152) (end 142.249 113.087) (width 0.25) (layer "F.Cu") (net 6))
 (segment (start 143.4925 110.01) (end 143.492 110.01) (width 0.25) (layer "F.Cu") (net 6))
 (segment (start 148.43 113.158) (end 148.43 113.67) (width 0.25) (layer "F.Cu") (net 6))
 (segment (start 147.342 110.427) (end 147.225 110.544) (width 0.25) (layer "F.Cu") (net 1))
 (segment (start 153.2225 108.37) (end 153.222 108.37) (width 0.25) (layer "F.Cu") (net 1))
 (segment (start 147.225 110.544) (end 147.342 110.427) (width 0.25) (layer "F.Cu") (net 1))
 (segment (start 156.3225 105.06) (end 156.322 105.06) (width 0.25) (layer "F.Cu") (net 1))
 (segment (start 152.57 109.861) (end 153.222 109.208) (width 0.25) (layer "F.Cu") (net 1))
 (segment (start 153.222 108.16) (end 156.322 105.06) (width 0.25) (layer "F.Cu") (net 1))
 (segment (start 147.225 110.544) (end 147.342 110.427) (width 0.25) (layer "F.Cu") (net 1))
 (segment (start 153.222 108.37) (end 153.222 108.16) (width 0.25) (layer "F.Cu") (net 1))
 (segment (start 153.222 109.208) (end 153.222 108.37) (width 0.25) (layer "F.Cu") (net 1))
 (segment (start 147.225 111.55) (end 147.225 110.544) (width 0.25) (layer "F.Cu") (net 1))
 (via (at 152.57 109.861) (size 0.7) (drill 0.3) (layers "F.Cu" "B.Cu") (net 1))
 (via (at 147.342 110.427) (size 0.7) (drill 0.3) (layers "F.Cu" "B.Cu") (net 1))
 (segment (start 147.342 110.427) (end 152.004 110.427) (width 0.25) (layer "B.Cu") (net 1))
 (segment (start 152.004 110.427) (end 152.57 109.861) (width 0.25) (layer "B.Cu") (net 1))
 (segment (start 155.798 94.05) (end 150.548 94.05) (width 0.25) (layer "F.Cu") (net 8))
 (segment (start 149.5 111.55) (end 151.736 109.314) (width 0.25) (layer "F.Cu") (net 8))
 (segment (start 150.5475 94.05) (end 150.548 94.05) (width 0.25) (layer "F.Cu") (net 8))
 (segment (start 151.617 95.6055) (end 150.548 94.5357) (width 0.25) (layer "F.Cu") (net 8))
 (segment (start 151.736 109.314) (end 151.736 95.724) (width 0.25) (layer "F.Cu") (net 8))
 (segment (start 151.736 95.724) (end 151.617 95.6055) (width 0.25) (layer "F.Cu") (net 8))
 (segment (start 150.548 94.5357) (end 150.548 94.05) (width 0.25) (layer "F.Cu") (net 8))
 (via (at 151.617 95.6055) (size 0.7) (drill 0.3) (layers "F.Cu" "B.Cu") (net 8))
 (segment (start 139.172 102.12) (end 145.687 95.6055) (width 0.25) (layer "B.Cu") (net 8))
 (segment (start 139.1725 102.12) (end 139.172 102.12) (width 0.25) (layer "B.Cu") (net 8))
 (segment (start 132.672 102.12) (end 139.172 102.12) (width 0.25) (layer "B.Cu") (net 8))
 (segment (start 145.687 95.6055) (end 151.617 95.6055) (width 0.25) (layer "B.Cu") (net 8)))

